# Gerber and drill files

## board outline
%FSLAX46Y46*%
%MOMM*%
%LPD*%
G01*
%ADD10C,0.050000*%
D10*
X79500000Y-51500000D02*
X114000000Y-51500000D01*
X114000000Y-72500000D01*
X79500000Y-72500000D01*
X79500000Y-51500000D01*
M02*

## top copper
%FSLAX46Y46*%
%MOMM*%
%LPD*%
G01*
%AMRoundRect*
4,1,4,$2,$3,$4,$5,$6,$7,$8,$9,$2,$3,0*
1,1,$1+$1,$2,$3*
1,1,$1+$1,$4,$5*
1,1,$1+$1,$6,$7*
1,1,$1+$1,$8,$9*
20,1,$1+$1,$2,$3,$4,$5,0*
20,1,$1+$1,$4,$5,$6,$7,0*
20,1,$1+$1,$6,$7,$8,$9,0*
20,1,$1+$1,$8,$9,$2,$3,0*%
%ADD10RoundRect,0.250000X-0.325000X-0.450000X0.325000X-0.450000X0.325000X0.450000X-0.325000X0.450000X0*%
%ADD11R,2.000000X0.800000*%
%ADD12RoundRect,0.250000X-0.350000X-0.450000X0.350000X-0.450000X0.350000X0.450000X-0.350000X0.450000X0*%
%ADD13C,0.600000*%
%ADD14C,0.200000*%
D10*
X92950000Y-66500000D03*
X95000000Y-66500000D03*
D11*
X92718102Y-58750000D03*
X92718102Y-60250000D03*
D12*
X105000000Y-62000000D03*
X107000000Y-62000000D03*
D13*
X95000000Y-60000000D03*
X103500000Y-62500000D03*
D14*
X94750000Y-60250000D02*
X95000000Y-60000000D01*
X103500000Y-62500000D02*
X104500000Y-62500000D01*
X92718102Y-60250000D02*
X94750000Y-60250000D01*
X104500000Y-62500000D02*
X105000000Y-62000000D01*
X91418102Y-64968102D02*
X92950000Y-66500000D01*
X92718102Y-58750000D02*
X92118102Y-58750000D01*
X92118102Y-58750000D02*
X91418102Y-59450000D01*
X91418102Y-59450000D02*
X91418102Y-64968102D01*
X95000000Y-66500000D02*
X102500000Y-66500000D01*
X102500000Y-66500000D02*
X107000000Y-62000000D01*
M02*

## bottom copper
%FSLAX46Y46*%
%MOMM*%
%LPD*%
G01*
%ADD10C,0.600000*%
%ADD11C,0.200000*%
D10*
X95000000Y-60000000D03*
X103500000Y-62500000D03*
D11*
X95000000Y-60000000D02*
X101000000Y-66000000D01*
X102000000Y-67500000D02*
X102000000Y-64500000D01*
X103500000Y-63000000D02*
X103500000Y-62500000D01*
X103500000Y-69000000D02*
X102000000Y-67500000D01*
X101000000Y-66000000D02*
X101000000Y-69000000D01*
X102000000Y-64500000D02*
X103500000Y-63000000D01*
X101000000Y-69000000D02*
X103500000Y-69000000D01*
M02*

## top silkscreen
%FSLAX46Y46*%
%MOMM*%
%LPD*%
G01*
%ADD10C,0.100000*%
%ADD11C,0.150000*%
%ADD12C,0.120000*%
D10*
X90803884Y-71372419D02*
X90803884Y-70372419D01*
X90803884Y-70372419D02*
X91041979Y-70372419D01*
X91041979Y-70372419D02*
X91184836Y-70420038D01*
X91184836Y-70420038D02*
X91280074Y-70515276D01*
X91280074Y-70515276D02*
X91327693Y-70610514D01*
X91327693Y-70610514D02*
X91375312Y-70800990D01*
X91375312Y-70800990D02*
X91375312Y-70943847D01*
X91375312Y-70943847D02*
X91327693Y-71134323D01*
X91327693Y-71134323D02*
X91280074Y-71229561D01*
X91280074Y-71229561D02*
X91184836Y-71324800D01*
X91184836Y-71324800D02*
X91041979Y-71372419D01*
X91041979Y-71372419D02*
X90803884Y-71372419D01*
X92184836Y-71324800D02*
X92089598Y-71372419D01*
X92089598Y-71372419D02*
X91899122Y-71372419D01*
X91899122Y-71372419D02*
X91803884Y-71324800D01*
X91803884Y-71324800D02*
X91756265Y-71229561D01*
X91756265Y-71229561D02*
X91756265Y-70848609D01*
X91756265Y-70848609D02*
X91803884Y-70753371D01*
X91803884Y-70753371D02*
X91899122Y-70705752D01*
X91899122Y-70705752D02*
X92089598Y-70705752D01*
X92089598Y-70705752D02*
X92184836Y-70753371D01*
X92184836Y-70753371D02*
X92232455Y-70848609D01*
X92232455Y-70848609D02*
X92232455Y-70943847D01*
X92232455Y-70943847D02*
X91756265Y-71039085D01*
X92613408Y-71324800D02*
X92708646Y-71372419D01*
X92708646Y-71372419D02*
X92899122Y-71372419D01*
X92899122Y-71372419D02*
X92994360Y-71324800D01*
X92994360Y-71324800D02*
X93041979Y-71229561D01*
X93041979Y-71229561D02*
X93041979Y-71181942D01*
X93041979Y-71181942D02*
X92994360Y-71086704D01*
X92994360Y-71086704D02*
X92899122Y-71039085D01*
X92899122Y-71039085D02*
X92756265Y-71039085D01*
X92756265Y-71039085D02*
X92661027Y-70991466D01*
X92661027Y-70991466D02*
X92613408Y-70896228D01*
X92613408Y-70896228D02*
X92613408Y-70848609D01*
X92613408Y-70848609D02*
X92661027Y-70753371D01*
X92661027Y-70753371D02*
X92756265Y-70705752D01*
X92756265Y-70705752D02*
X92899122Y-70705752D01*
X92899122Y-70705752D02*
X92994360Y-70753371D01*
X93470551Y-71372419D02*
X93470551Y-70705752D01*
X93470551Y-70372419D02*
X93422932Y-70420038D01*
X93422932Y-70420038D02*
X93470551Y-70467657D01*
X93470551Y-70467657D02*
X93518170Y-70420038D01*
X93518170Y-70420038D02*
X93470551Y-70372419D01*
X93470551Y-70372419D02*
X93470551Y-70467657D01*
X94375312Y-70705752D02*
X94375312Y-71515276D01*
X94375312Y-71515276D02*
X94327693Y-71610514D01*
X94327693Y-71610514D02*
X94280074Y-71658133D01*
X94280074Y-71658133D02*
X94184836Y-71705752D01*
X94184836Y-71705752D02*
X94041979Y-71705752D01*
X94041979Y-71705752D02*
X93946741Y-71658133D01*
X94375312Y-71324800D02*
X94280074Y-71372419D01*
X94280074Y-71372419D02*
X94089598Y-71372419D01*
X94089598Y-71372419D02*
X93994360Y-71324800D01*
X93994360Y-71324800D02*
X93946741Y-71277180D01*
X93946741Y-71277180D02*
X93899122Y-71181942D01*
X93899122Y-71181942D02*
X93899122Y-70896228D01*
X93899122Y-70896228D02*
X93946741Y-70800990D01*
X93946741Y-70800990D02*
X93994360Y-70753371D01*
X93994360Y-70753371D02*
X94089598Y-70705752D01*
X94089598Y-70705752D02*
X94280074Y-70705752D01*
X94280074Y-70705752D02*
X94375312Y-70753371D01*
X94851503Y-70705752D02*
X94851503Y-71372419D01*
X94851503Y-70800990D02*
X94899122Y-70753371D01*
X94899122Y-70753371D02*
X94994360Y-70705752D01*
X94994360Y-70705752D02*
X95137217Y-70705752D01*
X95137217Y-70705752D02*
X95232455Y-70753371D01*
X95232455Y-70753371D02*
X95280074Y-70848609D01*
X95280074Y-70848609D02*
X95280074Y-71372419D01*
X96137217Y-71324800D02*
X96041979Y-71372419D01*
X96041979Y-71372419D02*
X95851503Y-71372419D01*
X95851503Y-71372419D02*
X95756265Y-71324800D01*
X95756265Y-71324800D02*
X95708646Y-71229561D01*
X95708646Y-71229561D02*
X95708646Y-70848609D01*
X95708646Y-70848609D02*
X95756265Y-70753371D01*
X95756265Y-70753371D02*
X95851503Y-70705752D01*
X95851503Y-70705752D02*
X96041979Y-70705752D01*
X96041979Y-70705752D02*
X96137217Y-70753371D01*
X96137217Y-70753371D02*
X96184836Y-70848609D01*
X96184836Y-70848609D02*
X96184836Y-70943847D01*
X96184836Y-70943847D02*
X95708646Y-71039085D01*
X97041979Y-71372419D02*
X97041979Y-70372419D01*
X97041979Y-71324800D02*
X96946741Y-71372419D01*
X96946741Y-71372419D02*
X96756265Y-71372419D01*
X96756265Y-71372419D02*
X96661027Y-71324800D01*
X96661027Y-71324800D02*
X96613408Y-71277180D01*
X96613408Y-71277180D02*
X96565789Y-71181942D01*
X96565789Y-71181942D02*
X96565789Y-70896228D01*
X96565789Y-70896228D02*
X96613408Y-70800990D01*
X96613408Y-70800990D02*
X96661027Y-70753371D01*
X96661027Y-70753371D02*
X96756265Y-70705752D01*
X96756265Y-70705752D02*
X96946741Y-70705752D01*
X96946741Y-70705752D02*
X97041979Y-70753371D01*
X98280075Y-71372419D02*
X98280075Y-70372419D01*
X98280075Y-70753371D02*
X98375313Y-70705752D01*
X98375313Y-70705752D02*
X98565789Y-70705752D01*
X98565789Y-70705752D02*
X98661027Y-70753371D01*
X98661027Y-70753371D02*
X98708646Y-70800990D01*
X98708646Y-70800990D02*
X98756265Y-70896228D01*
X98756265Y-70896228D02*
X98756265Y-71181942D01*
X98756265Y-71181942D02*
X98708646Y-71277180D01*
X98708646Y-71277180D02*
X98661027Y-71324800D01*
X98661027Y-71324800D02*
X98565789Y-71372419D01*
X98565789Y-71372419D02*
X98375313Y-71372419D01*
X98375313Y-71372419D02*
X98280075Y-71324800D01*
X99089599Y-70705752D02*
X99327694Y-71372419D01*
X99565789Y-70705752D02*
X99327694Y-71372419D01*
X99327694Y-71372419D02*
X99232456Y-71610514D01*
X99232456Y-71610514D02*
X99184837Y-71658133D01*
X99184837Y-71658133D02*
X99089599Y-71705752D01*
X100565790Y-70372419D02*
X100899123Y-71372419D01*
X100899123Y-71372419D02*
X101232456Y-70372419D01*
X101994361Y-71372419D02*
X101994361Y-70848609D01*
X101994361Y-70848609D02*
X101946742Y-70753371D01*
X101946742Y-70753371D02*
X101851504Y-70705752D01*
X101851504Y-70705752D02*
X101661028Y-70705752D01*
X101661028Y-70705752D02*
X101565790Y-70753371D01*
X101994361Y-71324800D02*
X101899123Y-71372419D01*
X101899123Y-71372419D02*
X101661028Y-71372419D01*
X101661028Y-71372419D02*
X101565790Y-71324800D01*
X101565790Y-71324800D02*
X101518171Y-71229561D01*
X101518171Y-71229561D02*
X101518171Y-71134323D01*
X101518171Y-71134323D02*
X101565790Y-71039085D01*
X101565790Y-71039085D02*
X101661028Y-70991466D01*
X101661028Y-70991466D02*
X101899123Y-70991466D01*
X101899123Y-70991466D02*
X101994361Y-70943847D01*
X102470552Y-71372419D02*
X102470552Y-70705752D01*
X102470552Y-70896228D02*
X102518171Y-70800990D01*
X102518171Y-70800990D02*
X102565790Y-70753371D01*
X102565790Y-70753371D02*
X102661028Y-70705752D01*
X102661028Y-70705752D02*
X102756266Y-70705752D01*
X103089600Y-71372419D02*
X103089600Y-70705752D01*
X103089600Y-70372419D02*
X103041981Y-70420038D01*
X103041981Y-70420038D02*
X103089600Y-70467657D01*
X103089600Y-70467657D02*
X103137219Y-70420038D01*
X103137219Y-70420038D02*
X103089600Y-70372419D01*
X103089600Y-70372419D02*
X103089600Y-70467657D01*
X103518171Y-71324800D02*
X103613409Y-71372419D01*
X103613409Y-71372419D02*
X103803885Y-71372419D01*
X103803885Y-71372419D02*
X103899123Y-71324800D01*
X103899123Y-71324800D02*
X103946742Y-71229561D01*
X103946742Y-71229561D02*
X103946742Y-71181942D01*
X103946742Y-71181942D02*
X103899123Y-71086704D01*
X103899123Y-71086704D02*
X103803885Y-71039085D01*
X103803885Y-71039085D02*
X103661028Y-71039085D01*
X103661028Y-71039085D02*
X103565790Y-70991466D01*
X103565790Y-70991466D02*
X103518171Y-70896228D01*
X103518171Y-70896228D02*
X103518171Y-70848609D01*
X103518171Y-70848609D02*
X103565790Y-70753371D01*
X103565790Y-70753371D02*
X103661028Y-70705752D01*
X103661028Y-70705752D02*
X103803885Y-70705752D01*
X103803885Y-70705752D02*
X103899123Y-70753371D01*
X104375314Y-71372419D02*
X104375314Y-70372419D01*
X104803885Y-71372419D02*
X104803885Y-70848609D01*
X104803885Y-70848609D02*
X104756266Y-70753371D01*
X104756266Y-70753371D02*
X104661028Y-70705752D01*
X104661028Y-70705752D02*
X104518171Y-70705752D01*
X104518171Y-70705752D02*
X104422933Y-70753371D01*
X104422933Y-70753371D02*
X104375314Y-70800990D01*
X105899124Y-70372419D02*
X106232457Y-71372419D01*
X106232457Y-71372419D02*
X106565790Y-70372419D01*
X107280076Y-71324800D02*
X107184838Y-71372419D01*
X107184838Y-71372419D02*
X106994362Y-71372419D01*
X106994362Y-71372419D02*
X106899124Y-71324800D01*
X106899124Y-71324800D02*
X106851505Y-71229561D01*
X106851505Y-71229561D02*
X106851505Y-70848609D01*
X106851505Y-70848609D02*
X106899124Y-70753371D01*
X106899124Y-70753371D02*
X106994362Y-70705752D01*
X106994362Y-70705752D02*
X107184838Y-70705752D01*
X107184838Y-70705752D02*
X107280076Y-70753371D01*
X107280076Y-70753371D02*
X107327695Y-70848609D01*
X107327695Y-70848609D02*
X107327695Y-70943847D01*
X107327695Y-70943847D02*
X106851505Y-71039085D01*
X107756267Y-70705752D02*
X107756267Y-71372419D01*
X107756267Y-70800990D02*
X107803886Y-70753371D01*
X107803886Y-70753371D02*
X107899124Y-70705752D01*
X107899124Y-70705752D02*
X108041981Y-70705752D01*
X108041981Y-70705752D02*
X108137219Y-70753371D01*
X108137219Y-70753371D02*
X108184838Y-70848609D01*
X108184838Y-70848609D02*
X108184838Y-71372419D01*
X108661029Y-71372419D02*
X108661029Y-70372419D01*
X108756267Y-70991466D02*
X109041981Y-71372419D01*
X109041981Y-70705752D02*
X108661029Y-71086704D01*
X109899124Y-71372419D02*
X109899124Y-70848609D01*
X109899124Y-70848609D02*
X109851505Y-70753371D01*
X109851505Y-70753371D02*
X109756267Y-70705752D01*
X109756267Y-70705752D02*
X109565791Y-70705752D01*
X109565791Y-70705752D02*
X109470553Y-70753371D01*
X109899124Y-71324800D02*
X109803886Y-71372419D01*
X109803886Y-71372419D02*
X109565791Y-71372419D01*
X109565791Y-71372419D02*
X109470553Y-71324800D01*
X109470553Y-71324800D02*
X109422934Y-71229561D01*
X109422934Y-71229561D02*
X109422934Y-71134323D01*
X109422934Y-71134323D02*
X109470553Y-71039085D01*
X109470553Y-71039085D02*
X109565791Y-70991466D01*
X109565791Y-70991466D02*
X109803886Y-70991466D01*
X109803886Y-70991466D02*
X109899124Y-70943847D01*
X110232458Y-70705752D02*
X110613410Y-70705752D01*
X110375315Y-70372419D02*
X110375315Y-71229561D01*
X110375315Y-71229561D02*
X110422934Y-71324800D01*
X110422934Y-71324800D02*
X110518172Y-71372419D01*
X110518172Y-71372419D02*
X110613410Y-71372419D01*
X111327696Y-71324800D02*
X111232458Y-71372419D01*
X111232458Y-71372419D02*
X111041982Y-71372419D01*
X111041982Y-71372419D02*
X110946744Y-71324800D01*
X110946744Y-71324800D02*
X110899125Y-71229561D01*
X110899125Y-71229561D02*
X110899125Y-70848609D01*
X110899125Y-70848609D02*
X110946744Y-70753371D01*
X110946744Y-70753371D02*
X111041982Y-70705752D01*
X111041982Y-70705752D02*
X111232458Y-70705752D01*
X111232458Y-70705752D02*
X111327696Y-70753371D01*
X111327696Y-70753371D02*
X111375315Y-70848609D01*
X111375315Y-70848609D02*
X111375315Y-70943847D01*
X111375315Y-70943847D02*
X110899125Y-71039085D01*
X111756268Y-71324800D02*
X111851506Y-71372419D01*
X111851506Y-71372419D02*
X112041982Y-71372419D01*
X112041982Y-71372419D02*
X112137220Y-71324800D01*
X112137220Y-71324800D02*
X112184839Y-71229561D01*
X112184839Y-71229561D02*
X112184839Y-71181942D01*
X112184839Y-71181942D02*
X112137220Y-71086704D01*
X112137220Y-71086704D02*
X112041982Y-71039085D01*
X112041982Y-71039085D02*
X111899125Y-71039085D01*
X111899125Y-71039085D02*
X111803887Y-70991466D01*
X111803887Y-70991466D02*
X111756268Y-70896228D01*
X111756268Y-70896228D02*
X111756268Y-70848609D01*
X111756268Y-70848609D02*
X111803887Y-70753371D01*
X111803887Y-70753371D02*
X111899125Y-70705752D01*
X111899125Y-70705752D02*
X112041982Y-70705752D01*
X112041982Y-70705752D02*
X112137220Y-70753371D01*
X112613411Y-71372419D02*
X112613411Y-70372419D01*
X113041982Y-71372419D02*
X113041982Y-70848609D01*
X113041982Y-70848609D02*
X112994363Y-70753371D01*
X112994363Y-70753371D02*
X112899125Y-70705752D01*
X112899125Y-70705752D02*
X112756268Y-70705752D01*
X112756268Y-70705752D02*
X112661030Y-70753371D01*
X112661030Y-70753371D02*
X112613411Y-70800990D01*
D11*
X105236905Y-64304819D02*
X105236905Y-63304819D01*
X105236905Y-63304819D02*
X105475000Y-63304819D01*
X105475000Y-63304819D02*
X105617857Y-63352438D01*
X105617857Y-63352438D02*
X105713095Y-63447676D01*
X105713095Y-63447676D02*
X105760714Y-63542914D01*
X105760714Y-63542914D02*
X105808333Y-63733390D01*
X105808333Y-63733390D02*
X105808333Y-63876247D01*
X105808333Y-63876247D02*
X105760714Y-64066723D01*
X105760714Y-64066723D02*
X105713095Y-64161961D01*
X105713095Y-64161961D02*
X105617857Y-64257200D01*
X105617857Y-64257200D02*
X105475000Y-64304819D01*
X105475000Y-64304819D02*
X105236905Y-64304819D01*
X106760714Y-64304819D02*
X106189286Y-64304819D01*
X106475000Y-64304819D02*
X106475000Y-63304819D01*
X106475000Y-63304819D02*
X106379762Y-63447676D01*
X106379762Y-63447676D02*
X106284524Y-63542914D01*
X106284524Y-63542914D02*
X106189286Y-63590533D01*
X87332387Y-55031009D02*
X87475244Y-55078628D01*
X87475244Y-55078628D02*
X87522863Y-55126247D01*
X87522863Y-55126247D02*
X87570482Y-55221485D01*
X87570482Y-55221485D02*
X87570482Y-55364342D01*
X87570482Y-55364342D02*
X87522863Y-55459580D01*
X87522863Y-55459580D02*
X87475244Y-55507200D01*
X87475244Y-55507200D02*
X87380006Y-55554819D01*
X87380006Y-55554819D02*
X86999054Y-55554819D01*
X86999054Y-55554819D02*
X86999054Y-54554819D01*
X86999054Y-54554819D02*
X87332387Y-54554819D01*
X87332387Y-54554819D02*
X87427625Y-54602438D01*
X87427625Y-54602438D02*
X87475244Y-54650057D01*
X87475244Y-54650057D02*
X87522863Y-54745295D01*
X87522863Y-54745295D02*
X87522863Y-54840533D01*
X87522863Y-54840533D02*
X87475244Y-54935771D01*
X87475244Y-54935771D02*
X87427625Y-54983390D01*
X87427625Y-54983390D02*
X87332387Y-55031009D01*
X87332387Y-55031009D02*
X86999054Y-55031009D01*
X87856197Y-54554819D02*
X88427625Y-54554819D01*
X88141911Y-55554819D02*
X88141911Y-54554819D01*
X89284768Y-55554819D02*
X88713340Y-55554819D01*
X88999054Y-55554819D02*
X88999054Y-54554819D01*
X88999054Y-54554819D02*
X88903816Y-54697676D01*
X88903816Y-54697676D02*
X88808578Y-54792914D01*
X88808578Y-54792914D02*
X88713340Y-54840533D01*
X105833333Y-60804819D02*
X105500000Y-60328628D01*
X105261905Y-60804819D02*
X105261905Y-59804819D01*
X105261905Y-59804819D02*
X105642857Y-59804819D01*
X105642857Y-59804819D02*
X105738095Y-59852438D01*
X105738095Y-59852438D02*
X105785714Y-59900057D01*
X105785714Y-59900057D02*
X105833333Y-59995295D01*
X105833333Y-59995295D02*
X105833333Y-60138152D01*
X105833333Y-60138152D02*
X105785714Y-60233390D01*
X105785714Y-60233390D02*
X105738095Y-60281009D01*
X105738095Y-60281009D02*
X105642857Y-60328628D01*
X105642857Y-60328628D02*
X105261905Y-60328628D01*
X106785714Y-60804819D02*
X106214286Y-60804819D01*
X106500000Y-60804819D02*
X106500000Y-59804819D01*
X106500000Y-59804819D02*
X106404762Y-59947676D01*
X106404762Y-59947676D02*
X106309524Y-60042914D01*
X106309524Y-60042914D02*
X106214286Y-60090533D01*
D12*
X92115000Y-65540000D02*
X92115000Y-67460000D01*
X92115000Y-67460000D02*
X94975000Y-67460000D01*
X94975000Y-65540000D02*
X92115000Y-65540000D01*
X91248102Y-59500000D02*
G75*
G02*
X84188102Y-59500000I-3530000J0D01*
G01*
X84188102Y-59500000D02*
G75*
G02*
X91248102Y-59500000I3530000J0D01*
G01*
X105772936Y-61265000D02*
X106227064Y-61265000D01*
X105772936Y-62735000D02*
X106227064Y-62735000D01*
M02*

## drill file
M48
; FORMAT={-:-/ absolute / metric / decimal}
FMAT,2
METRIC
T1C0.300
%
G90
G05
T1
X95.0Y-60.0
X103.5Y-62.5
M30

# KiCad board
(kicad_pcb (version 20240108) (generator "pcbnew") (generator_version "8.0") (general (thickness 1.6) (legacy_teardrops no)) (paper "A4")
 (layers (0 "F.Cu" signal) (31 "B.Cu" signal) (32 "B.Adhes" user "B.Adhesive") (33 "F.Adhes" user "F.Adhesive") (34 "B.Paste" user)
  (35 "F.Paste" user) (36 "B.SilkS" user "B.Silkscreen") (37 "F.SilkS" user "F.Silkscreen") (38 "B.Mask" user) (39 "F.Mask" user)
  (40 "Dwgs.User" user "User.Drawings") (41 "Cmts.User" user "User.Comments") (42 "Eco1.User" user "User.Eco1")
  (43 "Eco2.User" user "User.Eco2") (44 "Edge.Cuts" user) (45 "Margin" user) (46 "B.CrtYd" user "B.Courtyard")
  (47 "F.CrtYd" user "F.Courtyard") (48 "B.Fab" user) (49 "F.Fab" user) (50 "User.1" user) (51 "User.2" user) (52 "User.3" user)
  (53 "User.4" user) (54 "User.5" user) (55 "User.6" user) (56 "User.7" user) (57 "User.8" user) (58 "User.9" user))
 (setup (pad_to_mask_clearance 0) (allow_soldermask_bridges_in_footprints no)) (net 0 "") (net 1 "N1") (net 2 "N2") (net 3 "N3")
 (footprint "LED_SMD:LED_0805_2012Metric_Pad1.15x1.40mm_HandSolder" (layer "F.Cu") (at 93.975 66.5)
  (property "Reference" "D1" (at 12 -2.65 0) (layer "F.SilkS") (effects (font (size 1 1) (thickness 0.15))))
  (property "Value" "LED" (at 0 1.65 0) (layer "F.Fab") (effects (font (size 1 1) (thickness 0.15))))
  (fp_line (start -1.86 -0.96) (end -1.86 0.96) (stroke (width 0.12) (type solid)) (layer "F.SilkS"))
  (fp_line (start -1.86 0.96) (end 1 0.96) (stroke (width 0.12) (type solid)) (layer "F.SilkS"))
  (fp_line (start 1 -0.96) (end -1.86 -0.96) (stroke (width 0.12) (type solid)) (layer "F.SilkS"))
  (pad "1" smd roundrect (at -1.025 0) (size 1.15 1.4) (layers "F.Cu" "F.Paste" "F.Mask") (roundrect_rratio 0.217391) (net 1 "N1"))
  (pad "2" smd roundrect (at 1.025 0) (size 1.15 1.4) (layers "F.Cu" "F.Paste" "F.Mask") (roundrect_rratio 0.217391) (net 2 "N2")))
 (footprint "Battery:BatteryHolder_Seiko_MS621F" (layer "F.Cu") (at 92.718102 59.5)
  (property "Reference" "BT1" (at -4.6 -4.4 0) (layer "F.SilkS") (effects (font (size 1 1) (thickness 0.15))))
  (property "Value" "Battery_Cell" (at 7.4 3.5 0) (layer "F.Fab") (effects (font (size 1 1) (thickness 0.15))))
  (fp_circle (center -5 0) (end -1.47 0) (stroke (width 0.12) (type solid)) (fill none) (layer "F.SilkS"))
  (pad "1" smd rect (at 0 -0.75) (size 2 0.8) (layers "F.Cu" "F.Paste" "F.Mask") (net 1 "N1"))
  (pad "2" smd rect (at 0 0.75) (size 2 0.8) (layers "F.Cu" "F.Paste" "F.Mask") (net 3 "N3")))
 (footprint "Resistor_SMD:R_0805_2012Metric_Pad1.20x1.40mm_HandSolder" (layer "F.Cu") (at 106 62)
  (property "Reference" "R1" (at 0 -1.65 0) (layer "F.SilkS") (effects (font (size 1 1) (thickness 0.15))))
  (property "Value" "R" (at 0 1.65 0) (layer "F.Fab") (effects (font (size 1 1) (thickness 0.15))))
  (fp_line (start -0.227064 -0.735) (end 0.227064 -0.735) (stroke (width 0.12) (type solid)) (layer "F.SilkS"))
  (fp_line (start -0.227064 0.735) (end 0.227064 0.735) (stroke (width 0.12) (type solid)) (layer "F.SilkS"))
  (pad "1" smd roundrect (at -1 0) (size 1.2 1.4) (layers "F.Cu" "F.Paste" "F.Mask") (roundrect_rratio 0.208333) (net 3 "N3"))
  (pad "2" smd roundrect (at 1 0) (size 1.2 1.4) (layers "F.Cu" "F.Paste" "F.Mask") (roundrect_rratio 0.208333) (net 2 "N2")))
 (gr_rect (start 79.5 51.5) (end 114 72.5) (stroke (width 0.05) (type default)) (fill none) (layer "Edge.Cuts"))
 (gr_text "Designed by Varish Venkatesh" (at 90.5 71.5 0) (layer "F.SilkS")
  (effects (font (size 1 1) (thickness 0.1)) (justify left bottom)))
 (segment (start 94.75 60.25) (end 95 60) (width 0.2) (layer "F.Cu") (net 3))
 (segment (start 103.5 62.5) (end 104.5 62.5) (width 0.2) (layer "F.Cu") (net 3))
 (segment (start 92.718102 60.25) (end 94.75 60.25) (width 0.2) (layer "F.Cu") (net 3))
 (segment (start 104.5 62.5) (end 105 62) (width 0.2) (layer "F.Cu") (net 3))
 (via (at 95 60) (size 0.6) (drill 0.3) (layers "F.Cu" "B.Cu") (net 3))
 (via (at 103.5 62.5) (size 0.6) (drill 0.3) (layers "F.Cu" "B.Cu") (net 3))
 (segment (start 95 60) (end 101 66) (width 0.2) (layer "B.Cu") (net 3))
 (segment (start 102 67.5) (end 102 64.5) (width 0.2) (layer "B.Cu") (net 3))
 (segment (start 103.5 63) (end 103.5 62.5) (width 0.2) (layer "B.Cu") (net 3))
 (segment (start 103.5 69) (end 102 67.5) (width 0.2) (layer "B.Cu") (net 3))
 (segment (start 101 66) (end 101 69) (width 0.2) (layer "B.Cu") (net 3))
 (segment (start 102 64.5) (end 103.5 63) (width 0.2) (layer "B.Cu") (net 3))
 (segment (start 101 69) (end 103.5 69) (width 0.2) (layer "B.Cu") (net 3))
 (segment (start 91.418102 64.968102) (end 92.95 66.5) (width 0.2) (layer "F.Cu") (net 1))
 (segment (start 92.718102 58.75) (end 92.118102 58.75) (width 0.2) (layer "F.Cu") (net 1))
 (segment (start 92.118102 58.75) (end 91.418102 59.45) (width 0.2) (layer "F.Cu") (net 1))
 (segment (start 91.418102 59.45) (end 91.418102 64.968102) (width 0.2) (layer "F.Cu") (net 1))
 (segment (start 95 66.5) (end 102.5 66.5) (width 0.2) (layer "F.Cu") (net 2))
 (segment (start 102.5 66.5) (end 107 62) (width 0.2) (layer "F.Cu") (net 2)))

